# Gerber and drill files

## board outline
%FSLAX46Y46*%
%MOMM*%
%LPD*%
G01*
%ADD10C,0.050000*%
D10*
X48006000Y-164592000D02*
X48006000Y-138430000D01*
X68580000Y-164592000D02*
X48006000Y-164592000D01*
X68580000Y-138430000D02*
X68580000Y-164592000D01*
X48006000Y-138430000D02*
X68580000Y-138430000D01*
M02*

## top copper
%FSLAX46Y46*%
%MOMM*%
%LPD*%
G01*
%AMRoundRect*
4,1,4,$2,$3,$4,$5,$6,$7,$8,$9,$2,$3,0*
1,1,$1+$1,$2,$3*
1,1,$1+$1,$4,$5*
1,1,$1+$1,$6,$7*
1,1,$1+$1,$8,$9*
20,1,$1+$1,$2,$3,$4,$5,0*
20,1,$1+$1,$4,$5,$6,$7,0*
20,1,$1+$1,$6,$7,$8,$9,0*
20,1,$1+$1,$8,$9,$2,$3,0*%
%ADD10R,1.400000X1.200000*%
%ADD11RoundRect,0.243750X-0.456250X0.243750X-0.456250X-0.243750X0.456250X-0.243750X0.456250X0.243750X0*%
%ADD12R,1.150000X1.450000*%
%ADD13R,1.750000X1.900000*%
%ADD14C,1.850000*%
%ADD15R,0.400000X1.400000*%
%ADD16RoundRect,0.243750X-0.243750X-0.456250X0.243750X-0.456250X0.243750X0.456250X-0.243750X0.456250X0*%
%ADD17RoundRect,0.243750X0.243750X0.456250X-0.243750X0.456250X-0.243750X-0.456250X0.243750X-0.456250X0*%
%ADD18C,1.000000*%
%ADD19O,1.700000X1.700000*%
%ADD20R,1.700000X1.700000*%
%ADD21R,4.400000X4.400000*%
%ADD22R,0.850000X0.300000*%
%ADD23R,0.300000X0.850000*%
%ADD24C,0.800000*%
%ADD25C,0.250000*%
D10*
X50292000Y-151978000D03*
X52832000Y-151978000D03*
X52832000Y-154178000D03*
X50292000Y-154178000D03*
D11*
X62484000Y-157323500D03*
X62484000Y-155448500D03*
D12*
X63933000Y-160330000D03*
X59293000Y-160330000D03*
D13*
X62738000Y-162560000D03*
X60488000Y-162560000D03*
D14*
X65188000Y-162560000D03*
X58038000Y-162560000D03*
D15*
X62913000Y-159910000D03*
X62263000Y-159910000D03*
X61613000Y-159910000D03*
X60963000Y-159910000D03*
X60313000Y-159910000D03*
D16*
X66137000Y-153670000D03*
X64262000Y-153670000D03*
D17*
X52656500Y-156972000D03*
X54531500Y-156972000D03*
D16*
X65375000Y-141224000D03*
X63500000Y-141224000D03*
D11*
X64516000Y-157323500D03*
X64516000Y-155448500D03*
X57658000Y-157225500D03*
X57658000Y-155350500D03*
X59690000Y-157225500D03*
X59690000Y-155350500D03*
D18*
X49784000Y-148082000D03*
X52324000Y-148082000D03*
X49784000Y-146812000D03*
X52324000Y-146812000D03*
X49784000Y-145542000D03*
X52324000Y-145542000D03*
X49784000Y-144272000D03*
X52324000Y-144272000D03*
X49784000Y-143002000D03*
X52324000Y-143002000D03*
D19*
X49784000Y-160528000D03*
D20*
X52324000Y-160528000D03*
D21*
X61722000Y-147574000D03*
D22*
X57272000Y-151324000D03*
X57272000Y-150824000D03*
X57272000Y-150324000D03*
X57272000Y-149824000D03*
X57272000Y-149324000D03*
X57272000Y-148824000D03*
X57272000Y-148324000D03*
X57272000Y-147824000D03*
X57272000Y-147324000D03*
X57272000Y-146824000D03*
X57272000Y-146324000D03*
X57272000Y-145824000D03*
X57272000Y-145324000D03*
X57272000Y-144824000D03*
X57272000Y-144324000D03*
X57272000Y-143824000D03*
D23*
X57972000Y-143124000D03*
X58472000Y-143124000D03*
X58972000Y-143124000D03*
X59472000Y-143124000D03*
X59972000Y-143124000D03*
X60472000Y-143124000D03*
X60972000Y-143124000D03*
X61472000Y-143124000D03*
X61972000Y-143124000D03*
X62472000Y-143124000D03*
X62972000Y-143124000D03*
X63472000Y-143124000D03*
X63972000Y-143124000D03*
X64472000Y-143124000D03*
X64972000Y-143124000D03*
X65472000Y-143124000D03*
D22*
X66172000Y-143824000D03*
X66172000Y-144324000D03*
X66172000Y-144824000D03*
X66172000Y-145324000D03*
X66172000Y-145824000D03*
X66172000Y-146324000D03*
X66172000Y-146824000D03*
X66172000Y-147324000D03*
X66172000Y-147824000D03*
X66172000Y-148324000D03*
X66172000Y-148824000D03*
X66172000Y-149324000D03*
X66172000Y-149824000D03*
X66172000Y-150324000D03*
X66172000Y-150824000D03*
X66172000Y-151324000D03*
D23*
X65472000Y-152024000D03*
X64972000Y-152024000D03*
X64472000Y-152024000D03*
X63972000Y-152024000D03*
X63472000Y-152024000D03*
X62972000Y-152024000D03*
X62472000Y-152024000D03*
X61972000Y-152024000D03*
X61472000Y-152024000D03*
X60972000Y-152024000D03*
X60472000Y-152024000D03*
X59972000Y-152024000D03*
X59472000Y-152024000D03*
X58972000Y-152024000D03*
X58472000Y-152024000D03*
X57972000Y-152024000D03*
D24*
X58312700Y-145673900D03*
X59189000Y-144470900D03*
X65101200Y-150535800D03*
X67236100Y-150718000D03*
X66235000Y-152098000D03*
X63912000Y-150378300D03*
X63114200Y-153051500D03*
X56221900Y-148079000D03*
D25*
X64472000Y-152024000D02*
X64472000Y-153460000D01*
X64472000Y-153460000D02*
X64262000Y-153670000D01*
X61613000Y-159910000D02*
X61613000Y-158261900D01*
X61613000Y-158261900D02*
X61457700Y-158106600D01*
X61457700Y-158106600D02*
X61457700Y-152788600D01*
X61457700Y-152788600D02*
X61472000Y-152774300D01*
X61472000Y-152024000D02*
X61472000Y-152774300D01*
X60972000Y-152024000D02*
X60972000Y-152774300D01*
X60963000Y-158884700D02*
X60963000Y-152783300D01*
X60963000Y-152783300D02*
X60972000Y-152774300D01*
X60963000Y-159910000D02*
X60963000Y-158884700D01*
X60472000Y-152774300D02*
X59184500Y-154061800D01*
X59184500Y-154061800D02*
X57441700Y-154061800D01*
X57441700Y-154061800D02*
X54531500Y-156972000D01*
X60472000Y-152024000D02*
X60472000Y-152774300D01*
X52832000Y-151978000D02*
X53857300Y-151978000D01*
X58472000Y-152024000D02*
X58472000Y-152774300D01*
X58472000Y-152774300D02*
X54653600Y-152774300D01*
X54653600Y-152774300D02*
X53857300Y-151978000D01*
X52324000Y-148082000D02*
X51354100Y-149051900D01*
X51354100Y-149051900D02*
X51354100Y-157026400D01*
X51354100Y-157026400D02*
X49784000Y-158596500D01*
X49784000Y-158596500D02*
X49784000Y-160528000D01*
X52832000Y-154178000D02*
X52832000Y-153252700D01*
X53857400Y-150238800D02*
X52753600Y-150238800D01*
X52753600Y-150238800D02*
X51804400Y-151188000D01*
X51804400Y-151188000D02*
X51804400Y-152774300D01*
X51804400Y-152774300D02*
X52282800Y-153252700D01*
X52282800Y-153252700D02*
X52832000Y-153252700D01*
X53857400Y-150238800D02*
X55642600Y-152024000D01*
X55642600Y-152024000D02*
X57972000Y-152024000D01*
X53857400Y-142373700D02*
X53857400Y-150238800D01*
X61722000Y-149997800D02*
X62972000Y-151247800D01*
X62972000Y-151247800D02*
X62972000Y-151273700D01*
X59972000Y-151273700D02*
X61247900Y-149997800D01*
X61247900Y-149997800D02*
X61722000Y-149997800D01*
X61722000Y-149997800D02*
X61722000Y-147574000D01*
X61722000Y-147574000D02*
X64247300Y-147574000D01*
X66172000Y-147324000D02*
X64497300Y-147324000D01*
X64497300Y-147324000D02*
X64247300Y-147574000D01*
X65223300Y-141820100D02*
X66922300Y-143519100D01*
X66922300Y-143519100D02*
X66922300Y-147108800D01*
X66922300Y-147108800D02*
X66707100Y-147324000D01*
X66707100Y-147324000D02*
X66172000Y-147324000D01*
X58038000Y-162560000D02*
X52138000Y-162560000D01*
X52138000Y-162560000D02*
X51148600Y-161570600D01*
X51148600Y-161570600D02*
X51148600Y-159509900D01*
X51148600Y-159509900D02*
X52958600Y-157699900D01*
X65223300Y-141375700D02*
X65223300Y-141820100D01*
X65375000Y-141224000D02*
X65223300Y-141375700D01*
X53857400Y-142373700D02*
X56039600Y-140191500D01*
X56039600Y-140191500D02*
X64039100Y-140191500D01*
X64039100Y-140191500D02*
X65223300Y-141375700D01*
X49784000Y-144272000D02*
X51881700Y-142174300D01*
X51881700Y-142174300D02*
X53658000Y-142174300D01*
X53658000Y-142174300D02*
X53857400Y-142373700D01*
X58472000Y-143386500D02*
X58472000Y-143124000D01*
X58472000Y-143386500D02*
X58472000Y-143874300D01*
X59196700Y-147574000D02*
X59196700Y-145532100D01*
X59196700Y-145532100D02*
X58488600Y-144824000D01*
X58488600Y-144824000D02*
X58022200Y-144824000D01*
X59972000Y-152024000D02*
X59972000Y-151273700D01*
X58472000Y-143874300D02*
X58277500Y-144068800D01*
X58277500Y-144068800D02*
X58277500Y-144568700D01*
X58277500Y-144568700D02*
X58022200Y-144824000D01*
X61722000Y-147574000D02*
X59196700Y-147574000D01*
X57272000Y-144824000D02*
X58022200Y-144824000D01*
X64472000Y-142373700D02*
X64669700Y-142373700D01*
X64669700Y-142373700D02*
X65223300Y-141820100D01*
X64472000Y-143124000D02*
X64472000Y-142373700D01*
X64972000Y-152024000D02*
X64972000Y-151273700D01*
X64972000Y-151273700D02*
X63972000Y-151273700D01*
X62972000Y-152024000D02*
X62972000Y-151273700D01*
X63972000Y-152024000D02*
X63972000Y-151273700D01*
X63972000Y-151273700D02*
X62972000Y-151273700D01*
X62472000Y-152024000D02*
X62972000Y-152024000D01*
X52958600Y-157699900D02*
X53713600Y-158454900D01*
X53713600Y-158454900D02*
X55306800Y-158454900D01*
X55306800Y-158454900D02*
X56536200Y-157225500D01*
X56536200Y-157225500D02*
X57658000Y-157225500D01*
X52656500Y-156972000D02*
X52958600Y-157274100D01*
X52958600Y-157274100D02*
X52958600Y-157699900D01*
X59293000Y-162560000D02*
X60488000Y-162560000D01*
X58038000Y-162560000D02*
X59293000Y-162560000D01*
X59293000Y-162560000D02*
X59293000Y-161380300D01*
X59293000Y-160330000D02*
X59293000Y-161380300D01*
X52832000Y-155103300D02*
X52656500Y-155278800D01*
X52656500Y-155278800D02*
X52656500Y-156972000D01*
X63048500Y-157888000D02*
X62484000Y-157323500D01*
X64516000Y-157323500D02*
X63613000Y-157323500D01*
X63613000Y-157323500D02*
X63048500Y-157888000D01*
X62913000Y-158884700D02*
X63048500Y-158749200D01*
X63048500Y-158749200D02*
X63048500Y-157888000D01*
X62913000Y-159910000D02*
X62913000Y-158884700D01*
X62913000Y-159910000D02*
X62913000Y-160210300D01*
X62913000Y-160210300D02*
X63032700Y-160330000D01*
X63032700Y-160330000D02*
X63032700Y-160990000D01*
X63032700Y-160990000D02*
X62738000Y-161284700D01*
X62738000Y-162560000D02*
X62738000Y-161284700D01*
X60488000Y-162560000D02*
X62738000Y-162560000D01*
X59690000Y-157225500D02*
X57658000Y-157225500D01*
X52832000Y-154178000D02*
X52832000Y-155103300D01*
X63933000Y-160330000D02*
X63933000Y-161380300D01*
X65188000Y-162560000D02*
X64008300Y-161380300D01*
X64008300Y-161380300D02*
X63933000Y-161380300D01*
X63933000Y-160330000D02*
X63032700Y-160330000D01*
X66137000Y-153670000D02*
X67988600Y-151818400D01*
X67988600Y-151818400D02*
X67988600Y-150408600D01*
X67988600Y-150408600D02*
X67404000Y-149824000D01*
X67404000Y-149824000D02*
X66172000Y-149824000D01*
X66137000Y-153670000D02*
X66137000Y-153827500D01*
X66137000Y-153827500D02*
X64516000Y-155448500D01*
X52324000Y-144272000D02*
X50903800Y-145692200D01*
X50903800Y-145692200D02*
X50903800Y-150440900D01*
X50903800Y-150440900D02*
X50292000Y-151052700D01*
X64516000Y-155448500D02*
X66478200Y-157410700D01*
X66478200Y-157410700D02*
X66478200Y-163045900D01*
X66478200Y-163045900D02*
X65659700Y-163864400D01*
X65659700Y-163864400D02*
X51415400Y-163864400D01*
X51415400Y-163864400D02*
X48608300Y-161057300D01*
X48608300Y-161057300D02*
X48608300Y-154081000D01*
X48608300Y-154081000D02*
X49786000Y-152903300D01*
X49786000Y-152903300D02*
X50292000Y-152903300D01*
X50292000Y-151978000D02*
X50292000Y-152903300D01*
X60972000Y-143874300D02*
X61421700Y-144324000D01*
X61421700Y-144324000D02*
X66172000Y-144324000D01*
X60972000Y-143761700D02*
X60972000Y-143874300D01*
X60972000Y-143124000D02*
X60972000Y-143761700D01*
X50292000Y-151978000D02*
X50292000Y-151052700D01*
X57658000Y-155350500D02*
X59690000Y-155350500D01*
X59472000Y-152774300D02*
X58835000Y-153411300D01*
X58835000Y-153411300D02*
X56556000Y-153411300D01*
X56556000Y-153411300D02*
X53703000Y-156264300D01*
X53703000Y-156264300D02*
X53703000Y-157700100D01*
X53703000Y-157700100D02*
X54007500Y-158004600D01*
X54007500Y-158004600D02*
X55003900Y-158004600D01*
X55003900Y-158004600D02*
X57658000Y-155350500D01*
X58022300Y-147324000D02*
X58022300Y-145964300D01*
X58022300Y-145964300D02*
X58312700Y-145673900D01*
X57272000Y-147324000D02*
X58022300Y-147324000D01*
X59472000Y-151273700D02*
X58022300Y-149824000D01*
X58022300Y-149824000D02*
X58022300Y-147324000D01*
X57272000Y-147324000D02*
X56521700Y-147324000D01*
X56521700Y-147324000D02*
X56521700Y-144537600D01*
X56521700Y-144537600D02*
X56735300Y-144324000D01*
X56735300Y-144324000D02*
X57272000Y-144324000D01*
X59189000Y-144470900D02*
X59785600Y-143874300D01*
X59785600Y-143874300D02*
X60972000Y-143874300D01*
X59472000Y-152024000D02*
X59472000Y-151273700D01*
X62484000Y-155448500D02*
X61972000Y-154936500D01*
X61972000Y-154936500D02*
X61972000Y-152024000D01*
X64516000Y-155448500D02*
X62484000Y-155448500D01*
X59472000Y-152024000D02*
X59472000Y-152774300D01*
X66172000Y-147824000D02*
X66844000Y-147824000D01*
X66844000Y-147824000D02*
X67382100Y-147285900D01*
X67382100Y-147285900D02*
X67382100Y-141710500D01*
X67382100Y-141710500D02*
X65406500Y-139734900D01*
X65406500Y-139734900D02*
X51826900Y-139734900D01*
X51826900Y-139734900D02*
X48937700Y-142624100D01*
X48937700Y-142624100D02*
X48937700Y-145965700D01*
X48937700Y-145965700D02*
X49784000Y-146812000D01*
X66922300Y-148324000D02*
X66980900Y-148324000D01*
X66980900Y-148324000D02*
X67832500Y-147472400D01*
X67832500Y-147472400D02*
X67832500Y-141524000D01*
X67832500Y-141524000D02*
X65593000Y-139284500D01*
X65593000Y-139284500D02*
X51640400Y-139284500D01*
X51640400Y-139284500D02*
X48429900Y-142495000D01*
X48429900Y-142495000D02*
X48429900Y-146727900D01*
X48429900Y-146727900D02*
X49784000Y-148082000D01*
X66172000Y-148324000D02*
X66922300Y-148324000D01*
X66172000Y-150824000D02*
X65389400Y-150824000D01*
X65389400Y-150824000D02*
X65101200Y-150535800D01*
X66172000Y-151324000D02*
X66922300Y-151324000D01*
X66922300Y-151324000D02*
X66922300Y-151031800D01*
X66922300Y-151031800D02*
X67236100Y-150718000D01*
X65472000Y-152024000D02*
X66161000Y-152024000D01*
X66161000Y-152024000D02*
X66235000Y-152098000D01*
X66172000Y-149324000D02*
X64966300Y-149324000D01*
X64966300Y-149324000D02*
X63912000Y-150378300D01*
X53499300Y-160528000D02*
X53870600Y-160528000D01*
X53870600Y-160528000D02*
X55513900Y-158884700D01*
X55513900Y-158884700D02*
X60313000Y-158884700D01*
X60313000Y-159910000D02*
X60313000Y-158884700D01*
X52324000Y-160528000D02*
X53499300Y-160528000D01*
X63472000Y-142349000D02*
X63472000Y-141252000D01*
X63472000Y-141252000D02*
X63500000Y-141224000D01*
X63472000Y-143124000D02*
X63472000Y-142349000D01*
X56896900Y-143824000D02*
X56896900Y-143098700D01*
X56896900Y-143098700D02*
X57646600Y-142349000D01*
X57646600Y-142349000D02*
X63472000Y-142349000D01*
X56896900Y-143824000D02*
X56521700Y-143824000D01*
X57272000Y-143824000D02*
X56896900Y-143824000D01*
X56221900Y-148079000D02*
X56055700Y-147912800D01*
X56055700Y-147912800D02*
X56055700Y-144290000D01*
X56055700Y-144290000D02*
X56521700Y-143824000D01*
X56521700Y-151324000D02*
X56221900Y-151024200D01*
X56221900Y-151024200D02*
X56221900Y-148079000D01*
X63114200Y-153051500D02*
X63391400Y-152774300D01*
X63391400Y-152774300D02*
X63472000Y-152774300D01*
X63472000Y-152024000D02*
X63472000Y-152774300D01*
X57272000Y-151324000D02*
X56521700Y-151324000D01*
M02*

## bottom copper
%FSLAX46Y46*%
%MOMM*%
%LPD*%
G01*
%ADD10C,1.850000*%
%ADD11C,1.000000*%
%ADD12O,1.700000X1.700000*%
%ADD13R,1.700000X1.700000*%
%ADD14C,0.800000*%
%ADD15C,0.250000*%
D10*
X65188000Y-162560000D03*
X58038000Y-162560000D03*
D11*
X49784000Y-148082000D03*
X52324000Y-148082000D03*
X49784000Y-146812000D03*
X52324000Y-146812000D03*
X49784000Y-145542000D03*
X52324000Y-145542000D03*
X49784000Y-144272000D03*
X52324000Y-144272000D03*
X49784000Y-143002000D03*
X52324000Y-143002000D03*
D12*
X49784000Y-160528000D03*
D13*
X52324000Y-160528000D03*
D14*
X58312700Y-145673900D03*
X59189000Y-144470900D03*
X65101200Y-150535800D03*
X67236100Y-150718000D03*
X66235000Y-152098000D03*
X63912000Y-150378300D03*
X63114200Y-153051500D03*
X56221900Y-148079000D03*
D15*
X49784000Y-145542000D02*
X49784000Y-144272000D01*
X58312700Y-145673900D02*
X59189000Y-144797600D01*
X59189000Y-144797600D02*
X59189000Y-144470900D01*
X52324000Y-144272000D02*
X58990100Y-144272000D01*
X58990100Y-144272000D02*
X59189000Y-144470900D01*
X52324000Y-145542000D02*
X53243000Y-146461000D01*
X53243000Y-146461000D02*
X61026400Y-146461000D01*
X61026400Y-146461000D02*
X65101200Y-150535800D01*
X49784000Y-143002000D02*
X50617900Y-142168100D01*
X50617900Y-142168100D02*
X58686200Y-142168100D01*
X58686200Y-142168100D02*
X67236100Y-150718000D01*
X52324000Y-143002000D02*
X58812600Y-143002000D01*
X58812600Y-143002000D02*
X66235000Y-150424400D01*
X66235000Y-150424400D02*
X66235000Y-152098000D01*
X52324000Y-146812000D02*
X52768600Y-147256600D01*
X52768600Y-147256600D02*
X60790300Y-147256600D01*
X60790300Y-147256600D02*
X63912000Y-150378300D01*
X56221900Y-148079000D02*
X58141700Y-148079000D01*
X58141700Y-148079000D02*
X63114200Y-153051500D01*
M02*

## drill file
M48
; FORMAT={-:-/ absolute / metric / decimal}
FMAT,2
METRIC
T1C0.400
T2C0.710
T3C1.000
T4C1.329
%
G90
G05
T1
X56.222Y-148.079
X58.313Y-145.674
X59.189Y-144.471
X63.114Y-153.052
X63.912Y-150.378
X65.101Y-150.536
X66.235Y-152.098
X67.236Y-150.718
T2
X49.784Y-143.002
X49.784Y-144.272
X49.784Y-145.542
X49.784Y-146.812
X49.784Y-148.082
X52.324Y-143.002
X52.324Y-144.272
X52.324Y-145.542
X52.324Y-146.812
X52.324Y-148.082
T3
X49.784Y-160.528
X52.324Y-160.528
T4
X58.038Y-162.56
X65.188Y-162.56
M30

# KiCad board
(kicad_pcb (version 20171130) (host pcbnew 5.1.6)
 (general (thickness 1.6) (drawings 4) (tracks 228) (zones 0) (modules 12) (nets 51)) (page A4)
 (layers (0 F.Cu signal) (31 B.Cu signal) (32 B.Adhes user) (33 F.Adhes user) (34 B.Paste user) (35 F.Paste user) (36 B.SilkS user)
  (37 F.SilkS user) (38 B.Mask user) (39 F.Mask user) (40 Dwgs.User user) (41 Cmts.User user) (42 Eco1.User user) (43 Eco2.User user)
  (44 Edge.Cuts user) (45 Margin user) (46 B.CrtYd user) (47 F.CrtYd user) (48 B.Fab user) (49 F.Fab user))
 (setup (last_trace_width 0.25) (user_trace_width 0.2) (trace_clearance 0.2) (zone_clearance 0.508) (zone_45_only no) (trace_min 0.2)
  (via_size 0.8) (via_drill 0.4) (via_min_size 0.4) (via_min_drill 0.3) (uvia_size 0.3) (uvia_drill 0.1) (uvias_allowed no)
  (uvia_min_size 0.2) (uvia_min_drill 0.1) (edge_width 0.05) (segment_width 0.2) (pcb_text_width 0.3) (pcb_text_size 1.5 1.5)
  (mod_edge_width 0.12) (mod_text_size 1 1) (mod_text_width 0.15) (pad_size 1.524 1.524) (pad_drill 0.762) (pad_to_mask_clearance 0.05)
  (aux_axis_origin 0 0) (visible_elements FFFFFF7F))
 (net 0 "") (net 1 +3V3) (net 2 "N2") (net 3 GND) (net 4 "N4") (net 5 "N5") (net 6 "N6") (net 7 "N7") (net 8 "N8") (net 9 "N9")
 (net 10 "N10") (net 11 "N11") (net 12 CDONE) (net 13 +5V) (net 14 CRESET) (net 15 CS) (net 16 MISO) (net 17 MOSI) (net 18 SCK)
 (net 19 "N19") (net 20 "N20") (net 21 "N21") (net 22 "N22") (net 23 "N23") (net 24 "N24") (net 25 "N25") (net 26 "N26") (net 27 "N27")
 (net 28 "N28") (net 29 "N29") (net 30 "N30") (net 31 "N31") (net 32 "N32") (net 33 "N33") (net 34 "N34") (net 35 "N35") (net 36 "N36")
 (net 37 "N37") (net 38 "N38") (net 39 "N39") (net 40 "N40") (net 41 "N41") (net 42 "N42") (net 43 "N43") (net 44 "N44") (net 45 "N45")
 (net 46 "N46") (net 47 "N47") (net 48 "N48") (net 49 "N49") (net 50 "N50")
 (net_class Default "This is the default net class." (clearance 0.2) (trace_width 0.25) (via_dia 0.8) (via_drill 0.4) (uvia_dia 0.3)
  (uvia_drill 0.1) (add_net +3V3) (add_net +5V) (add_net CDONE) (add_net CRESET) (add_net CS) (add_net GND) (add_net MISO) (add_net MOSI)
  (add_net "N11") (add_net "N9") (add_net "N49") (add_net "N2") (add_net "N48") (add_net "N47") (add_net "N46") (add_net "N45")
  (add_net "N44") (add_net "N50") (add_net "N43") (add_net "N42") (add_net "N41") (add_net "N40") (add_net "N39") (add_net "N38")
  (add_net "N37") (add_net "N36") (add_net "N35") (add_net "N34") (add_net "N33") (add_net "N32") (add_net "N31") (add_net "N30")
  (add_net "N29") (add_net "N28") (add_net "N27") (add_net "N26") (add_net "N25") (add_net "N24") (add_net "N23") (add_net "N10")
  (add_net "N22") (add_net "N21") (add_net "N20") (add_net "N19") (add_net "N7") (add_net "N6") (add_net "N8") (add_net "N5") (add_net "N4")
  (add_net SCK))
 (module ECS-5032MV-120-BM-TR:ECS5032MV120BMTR (layer F.Cu) (at 51.562 153.078)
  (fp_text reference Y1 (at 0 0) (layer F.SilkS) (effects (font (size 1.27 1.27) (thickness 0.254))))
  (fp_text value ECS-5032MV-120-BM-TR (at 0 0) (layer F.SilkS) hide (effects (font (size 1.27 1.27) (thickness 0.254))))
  (pad 4 smd rect (at -1.27 -1.1 90) (size 1.2 1.4) (layers F.Cu F.Paste F.Mask) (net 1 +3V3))
  (pad 3 smd rect (at 1.27 -1.1 90) (size 1.2 1.4) (layers F.Cu F.Paste F.Mask) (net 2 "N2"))
  (pad 2 smd rect (at 1.27 1.1 90) (size 1.2 1.4) (layers F.Cu F.Paste F.Mask) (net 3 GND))
  (pad 1 smd rect (at -1.27 1.1 90) (size 1.2 1.4) (layers F.Cu F.Paste F.Mask) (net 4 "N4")))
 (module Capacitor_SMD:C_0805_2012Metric (layer F.Cu) (at 62.484 156.386 270)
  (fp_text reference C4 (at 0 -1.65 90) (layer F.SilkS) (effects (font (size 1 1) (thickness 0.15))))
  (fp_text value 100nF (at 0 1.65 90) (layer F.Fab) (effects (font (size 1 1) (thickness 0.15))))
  (pad 2 smd roundrect (at 0.9375 0 270) (size 0.975 1.4) (layers F.Cu F.Paste F.Mask) (roundrect_rratio 0.25) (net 3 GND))
  (pad 1 smd roundrect (at -0.9375 0 270) (size 0.975 1.4) (layers F.Cu F.Paste F.Mask) (roundrect_rratio 0.25) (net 1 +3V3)))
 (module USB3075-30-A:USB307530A (layer F.Cu) (at 61.613 162.56)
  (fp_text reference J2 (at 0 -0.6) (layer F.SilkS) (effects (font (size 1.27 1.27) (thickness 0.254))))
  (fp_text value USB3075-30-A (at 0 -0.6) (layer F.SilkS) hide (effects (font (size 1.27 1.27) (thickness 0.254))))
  (pad MP4 smd rect (at 2.32 -2.23) (size 1.15 1.45) (layers F.Cu F.Paste F.Mask) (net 3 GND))
  (pad MP3 smd rect (at -2.32 -2.23) (size 1.15 1.45) (layers F.Cu F.Paste F.Mask) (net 3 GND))
  (pad MP2 smd rect (at 1.125 0) (size 1.75 1.9) (layers F.Cu F.Paste F.Mask) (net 3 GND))
  (pad MP1 smd rect (at -1.125 0) (size 1.75 1.9) (layers F.Cu F.Paste F.Mask) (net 3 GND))
  (pad MH2 thru_hole circle (at 3.575 0) (size 1.85 1.85) (drill 1.3285) (layers *.Cu *.Mask) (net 3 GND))
  (pad MH1 thru_hole circle (at -3.575 0) (size 1.85 1.85) (drill 1.3285) (layers *.Cu *.Mask) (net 3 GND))
  (pad 5 smd rect (at 1.3 -2.65) (size 0.4 1.4) (layers F.Cu F.Paste F.Mask) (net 3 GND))
  (pad 4 smd rect (at 0.65 -2.65) (size 0.4 1.4) (layers F.Cu F.Paste F.Mask) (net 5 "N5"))
  (pad 3 smd rect (at 0 -2.65) (size 0.4 1.4) (layers F.Cu F.Paste F.Mask) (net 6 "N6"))
  (pad 2 smd rect (at -0.65 -2.65) (size 0.4 1.4) (layers F.Cu F.Paste F.Mask) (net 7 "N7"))
  (pad 1 smd rect (at -1.3 -2.65) (size 0.4 1.4) (layers F.Cu F.Paste F.Mask) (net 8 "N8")))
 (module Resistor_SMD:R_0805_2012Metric (layer F.Cu) (at 65.1995 153.67)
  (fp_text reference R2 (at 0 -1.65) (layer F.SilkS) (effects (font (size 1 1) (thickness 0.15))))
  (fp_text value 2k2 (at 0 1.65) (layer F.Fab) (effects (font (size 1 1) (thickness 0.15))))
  (pad 2 smd roundrect (at 0.9375 0) (size 0.975 1.4) (layers F.Cu F.Paste F.Mask) (roundrect_rratio 0.25) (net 1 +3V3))
  (pad 1 smd roundrect (at -0.9375 0) (size 0.975 1.4) (layers F.Cu F.Paste F.Mask) (roundrect_rratio 0.25) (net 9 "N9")))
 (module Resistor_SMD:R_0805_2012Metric (layer F.Cu) (at 53.594 156.972 180)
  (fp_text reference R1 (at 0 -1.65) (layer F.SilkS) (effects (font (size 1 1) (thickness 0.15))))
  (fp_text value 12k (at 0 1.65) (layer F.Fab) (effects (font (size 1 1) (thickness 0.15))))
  (pad 2 smd roundrect (at 0.9375 0 180) (size 0.975 1.4) (layers F.Cu F.Paste F.Mask) (roundrect_rratio 0.25) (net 3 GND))
  (pad 1 smd roundrect (at -0.9375 0 180) (size 0.975 1.4) (layers F.Cu F.Paste F.Mask) (roundrect_rratio 0.25) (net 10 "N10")))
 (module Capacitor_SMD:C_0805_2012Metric (layer F.Cu) (at 64.4375 141.224)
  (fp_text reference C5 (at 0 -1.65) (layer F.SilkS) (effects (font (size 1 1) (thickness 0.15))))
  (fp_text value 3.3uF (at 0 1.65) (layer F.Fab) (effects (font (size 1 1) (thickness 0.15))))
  (pad 2 smd roundrect (at 0.9375 0) (size 0.975 1.4) (layers F.Cu F.Paste F.Mask) (roundrect_rratio 0.25) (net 3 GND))
  (pad 1 smd roundrect (at -0.9375 0) (size 0.975 1.4) (layers F.Cu F.Paste F.Mask) (roundrect_rratio 0.25) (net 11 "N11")))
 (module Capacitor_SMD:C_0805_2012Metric (layer F.Cu) (at 64.516 156.386 270)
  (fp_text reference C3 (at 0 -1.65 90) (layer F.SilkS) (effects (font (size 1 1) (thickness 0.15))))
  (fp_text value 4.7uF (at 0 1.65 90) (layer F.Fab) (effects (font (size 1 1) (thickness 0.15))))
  (pad 2 smd roundrect (at 0.9375 0 270) (size 0.975 1.4) (layers F.Cu F.Paste F.Mask) (roundrect_rratio 0.25) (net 3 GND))
  (pad 1 smd roundrect (at -0.9375 0 270) (size 0.975 1.4) (layers F.Cu F.Paste F.Mask) (roundrect_rratio 0.25) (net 1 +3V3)))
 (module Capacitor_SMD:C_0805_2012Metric (layer F.Cu) (at 57.658 156.288 270)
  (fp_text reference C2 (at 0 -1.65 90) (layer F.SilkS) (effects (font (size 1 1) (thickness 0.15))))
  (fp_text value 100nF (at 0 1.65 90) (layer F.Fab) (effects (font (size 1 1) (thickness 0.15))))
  (pad 2 smd roundrect (at 0.9375 0 270) (size 0.975 1.4) (layers F.Cu F.Paste F.Mask) (roundrect_rratio 0.25) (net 3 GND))
  (pad 1 smd roundrect (at -0.9375 0 270) (size 0.975 1.4) (layers F.Cu F.Paste F.Mask) (roundrect_rratio 0.25) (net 1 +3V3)))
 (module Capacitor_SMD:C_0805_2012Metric (layer F.Cu) (at 59.69 156.288 270)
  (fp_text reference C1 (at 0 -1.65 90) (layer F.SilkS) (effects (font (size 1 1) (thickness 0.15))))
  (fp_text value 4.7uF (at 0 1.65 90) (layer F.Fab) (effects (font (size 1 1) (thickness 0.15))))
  (pad 2 smd roundrect (at 0.9375 0 270) (size 0.975 1.4) (layers F.Cu F.Paste F.Mask) (roundrect_rratio 0.25) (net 3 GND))
  (pad 1 smd roundrect (at -0.9375 0 270) (size 0.975 1.4) (layers F.Cu F.Paste F.Mask) (roundrect_rratio 0.25) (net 1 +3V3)))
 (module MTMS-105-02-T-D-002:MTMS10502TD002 (layer B.Cu) (at 52.324 143.002 270)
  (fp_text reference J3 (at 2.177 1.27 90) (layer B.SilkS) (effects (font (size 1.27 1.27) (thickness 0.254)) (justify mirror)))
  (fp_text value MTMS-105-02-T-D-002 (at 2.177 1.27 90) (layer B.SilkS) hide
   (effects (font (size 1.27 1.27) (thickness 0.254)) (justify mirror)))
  (pad 10 thru_hole circle (at 5.08 2.54 270) (size 1 1) (drill 0.71) (layers *.Cu *.Mask) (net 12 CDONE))
  (pad 9 thru_hole circle (at 5.08 0 270) (size 1 1) (drill 0.71) (layers *.Cu *.Mask) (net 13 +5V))
  (pad 8 thru_hole circle (at 3.81 2.54 270) (size 1 1) (drill 0.71) (layers *.Cu *.Mask) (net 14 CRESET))
  (pad 7 thru_hole circle (at 3.81 0 270) (size 1 1) (drill 0.71) (layers *.Cu *.Mask) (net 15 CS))
  (pad 6 thru_hole circle (at 2.54 2.54 270) (size 1 1) (drill 0.71) (layers *.Cu *.Mask) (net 3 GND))
  (pad 5 thru_hole circle (at 2.54 0 270) (size 1 1) (drill 0.71) (layers *.Cu *.Mask) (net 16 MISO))
  (pad 4 thru_hole circle (at 1.27 2.54 270) (size 1 1) (drill 0.71) (layers *.Cu *.Mask) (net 3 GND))
  (pad 3 thru_hole circle (at 1.27 0 270) (size 1 1) (drill 0.71) (layers *.Cu *.Mask) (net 1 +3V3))
  (pad 2 thru_hole circle (at 0 2.54 270) (size 1 1) (drill 0.71) (layers *.Cu *.Mask) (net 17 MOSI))
  (pad 1 thru_hole circle (at 0 0 270) (size 1 1) (drill 0.71) (layers *.Cu *.Mask) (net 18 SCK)))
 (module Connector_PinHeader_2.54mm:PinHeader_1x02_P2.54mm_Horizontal (layer F.Cu) (at 52.324 160.528 270)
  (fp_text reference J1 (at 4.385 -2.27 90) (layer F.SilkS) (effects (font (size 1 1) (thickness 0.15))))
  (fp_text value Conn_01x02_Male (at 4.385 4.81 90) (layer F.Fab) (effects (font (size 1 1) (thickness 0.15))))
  (pad 2 thru_hole oval (at 0 2.54 270) (size 1.7 1.7) (drill 1) (layers *.Cu *.Mask) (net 13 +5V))
  (pad 1 thru_hole rect (at 0 0 270) (size 1.7 1.7) (drill 1) (layers *.Cu *.Mask) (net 8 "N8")))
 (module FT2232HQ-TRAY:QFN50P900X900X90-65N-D (layer F.Cu) (at 61.722 147.574 90)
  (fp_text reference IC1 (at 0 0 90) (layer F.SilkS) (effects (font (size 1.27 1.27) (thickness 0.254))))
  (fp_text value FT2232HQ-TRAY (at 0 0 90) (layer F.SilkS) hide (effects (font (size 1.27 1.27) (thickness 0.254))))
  (pad 65 smd rect (at 0 0 90) (size 4.4 4.4) (layers F.Cu F.Paste F.Mask) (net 3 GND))
  (pad 64 smd rect (at -3.75 -4.45 90) (size 0.3 0.85) (layers F.Cu F.Paste F.Mask) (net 11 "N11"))
  (pad 63 smd rect (at -3.25 -4.45 90) (size 0.3 0.85) (layers F.Cu F.Paste F.Mask) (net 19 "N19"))
  (pad 62 smd rect (at -2.75 -4.45 90) (size 0.3 0.85) (layers F.Cu F.Paste F.Mask) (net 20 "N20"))
  (pad 61 smd rect (at -2.25 -4.45 90) (size 0.3 0.85) (layers F.Cu F.Paste F.Mask) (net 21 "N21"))
  (pad 60 smd rect (at -1.75 -4.45 90) (size 0.3 0.85) (layers F.Cu F.Paste F.Mask) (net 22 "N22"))
  (pad 59 smd rect (at -1.25 -4.45 90) (size 0.3 0.85) (layers F.Cu F.Paste F.Mask) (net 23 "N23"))
  (pad 58 smd rect (at -0.75 -4.45 90) (size 0.3 0.85) (layers F.Cu F.Paste F.Mask) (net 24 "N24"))
  (pad 57 smd rect (at -0.25 -4.45 90) (size 0.3 0.85) (layers F.Cu F.Paste F.Mask) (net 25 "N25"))
  (pad 56 smd rect (at 0.25 -4.45 90) (size 0.3 0.85) (layers F.Cu F.Paste F.Mask) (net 1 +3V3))
  (pad 55 smd rect (at 0.75 -4.45 90) (size 0.3 0.85) (layers F.Cu F.Paste F.Mask) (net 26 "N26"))
  (pad 54 smd rect (at 1.25 -4.45 90) (size 0.3 0.85) (layers F.Cu F.Paste F.Mask) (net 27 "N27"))
  (pad 53 smd rect (at 1.75 -4.45 90) (size 0.3 0.85) (layers F.Cu F.Paste F.Mask) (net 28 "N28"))
  (pad 52 smd rect (at 2.25 -4.45 90) (size 0.3 0.85) (layers F.Cu F.Paste F.Mask) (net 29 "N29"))
  (pad 51 smd rect (at 2.75 -4.45 90) (size 0.3 0.85) (layers F.Cu F.Paste F.Mask) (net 3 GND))
  (pad 50 smd rect (at 3.25 -4.45 90) (size 0.3 0.85) (layers F.Cu F.Paste F.Mask) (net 1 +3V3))
  (pad 49 smd rect (at 3.75 -4.45 90) (size 0.3 0.85) (layers F.Cu F.Paste F.Mask) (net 11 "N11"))
  (pad 48 smd rect (at 4.45 -3.75 180) (size 0.3 0.85) (layers F.Cu F.Paste F.Mask) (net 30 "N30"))
  (pad 47 smd rect (at 4.45 -3.25 180) (size 0.3 0.85) (layers F.Cu F.Paste F.Mask) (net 3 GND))
  (pad 46 smd rect (at 4.45 -2.75 180) (size 0.3 0.85) (layers F.Cu F.Paste F.Mask) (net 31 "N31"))
  (pad 45 smd rect (at 4.45 -2.25 180) (size 0.3 0.85) (layers F.Cu F.Paste F.Mask) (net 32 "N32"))
  (pad 44 smd rect (at 4.45 -1.75 180) (size 0.3 0.85) (layers F.Cu F.Paste F.Mask) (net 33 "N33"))
  (pad 43 smd rect (at 4.45 -1.25 180) (size 0.3 0.85) (layers F.Cu F.Paste F.Mask) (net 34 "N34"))
  (pad 42 smd rect (at 4.45 -0.75 180) (size 0.3 0.85) (layers F.Cu F.Paste F.Mask) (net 1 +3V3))
  (pad 41 smd rect (at 4.45 -0.25 180) (size 0.3 0.85) (layers F.Cu F.Paste F.Mask) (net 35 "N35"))
  (pad 40 smd rect (at 4.45 0.25 180) (size 0.3 0.85) (layers F.Cu F.Paste F.Mask) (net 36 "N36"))
  (pad 39 smd rect (at 4.45 0.75 180) (size 0.3 0.85) (layers F.Cu F.Paste F.Mask) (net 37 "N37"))
  (pad 38 smd rect (at 4.45 1.25 180) (size 0.3 0.85) (layers F.Cu F.Paste F.Mask) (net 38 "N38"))
  (pad 37 smd rect (at 4.45 1.75 180) (size 0.3 0.85) (layers F.Cu F.Paste F.Mask) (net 11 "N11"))
  (pad 36 smd rect (at 4.45 2.25 180) (size 0.3 0.85) (layers F.Cu F.Paste F.Mask) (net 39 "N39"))
  (pad 35 smd rect (at 4.45 2.75 180) (size 0.3 0.85) (layers F.Cu F.Paste F.Mask) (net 3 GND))
  (pad 34 smd rect (at 4.45 3.25 180) (size 0.3 0.85) (layers F.Cu F.Paste F.Mask) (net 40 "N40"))
  (pad 33 smd rect (at 4.45 3.75 180) (size 0.3 0.85) (layers F.Cu F.Paste F.Mask) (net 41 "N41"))
  (pad 32 smd rect (at 3.75 4.45 90) (size 0.3 0.85) (layers F.Cu F.Paste F.Mask) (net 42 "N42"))
  (pad 31 smd rect (at 3.25 4.45 90) (size 0.3 0.85) (layers F.Cu F.Paste F.Mask) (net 1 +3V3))
  (pad 30 smd rect (at 2.75 4.45 90) (size 0.3 0.85) (layers F.Cu F.Paste F.Mask) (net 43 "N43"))
  (pad 29 smd rect (at 2.25 4.45 90) (size 0.3 0.85) (layers F.Cu F.Paste F.Mask) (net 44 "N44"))
  (pad 28 smd rect (at 1.75 4.45 90) (size 0.3 0.85) (layers F.Cu F.Paste F.Mask) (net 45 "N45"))
  (pad 27 smd rect (at 1.25 4.45 90) (size 0.3 0.85) (layers F.Cu F.Paste F.Mask) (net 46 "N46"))
  (pad 26 smd rect (at 0.75 4.45 90) (size 0.3 0.85) (layers F.Cu F.Paste F.Mask) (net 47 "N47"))
  (pad 25 smd rect (at 0.25 4.45 90) (size 0.3 0.85) (layers F.Cu F.Paste F.Mask) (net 3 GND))
  (pad 24 smd rect (at -0.25 4.45 90) (size 0.3 0.85) (layers F.Cu F.Paste F.Mask) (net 14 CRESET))
  (pad 23 smd rect (at -0.75 4.45 90) (size 0.3 0.85) (layers F.Cu F.Paste F.Mask) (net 12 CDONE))
  (pad 22 smd rect (at -1.25 4.45 90) (size 0.3 0.85) (layers F.Cu F.Paste F.Mask) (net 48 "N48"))
  (pad 21 smd rect (at -1.75 4.45 90) (size 0.3 0.85) (layers F.Cu F.Paste F.Mask) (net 15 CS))
  (pad 20 smd rect (at -2.25 4.45 90) (size 0.3 0.85) (layers F.Cu F.Paste F.Mask) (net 1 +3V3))
  (pad 19 smd rect (at -2.75 4.45 90) (size 0.3 0.85) (layers F.Cu F.Paste F.Mask) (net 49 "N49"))
  (pad 18 smd rect (at -3.25 4.45 90) (size 0.3 0.85) (layers F.Cu F.Paste F.Mask) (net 16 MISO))
  (pad 17 smd rect (at -3.75 4.45 90) (size 0.3 0.85) (layers F.Cu F.Paste F.Mask) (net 17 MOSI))
  (pad 16 smd rect (at -4.45 3.75 180) (size 0.3 0.85) (layers F.Cu F.Paste F.Mask) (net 18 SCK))
  (pad 15 smd rect (at -4.45 3.25 180) (size 0.3 0.85) (layers F.Cu F.Paste F.Mask) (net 3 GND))
  (pad 14 smd rect (at -4.45 2.75 180) (size 0.3 0.85) (layers F.Cu F.Paste F.Mask) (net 9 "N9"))
  (pad 13 smd rect (at -4.45 2.25 180) (size 0.3 0.85) (layers F.Cu F.Paste F.Mask) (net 3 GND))
  (pad 12 smd rect (at -4.45 1.75 180) (size 0.3 0.85) (layers F.Cu F.Paste F.Mask) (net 11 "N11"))
  (pad 11 smd rect (at -4.45 1.25 180) (size 0.3 0.85) (layers F.Cu F.Paste F.Mask) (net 3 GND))
  (pad 10 smd rect (at -4.45 0.75 180) (size 0.3 0.85) (layers F.Cu F.Paste F.Mask) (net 3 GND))
  (pad 9 smd rect (at -4.45 0.25 180) (size 0.3 0.85) (layers F.Cu F.Paste F.Mask) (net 1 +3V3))
  (pad 8 smd rect (at -4.45 -0.25 180) (size 0.3 0.85) (layers F.Cu F.Paste F.Mask) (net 6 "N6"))
  (pad 7 smd rect (at -4.45 -0.75 180) (size 0.3 0.85) (layers F.Cu F.Paste F.Mask) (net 7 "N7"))
  (pad 6 smd rect (at -4.45 -1.25 180) (size 0.3 0.85) (layers F.Cu F.Paste F.Mask) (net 10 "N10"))
  (pad 5 smd rect (at -4.45 -1.75 180) (size 0.3 0.85) (layers F.Cu F.Paste F.Mask) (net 3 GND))
  (pad 4 smd rect (at -4.45 -2.25 180) (size 0.3 0.85) (layers F.Cu F.Paste F.Mask) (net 1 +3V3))
  (pad 3 smd rect (at -4.45 -2.75 180) (size 0.3 0.85) (layers F.Cu F.Paste F.Mask) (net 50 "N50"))
  (pad 2 smd rect (at -4.45 -3.25 180) (size 0.3 0.85) (layers F.Cu F.Paste F.Mask) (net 2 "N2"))
  (pad 1 smd rect (at -4.45 -3.75 180) (size 0.3 0.85) (layers F.Cu F.Paste F.Mask) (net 3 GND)))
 (gr_line (start 48.006 164.592) (end 48.006 138.43) (layer Edge.Cuts) (width 0.05))
 (gr_line (start 68.58 164.592) (end 48.006 164.592) (layer Edge.Cuts) (width 0.05))
 (gr_line (start 68.58 138.43) (end 68.58 164.592) (layer Edge.Cuts) (width 0.05))
 (gr_line (start 48.006 138.43) (end 68.58 138.43) (layer Edge.Cuts) (width 0.05))
 (segment (start 64.472 152.024) (end 64.472 153.46) (width 0.25) (layer F.Cu) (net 9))
 (segment (start 64.472 153.46) (end 64.262 153.67) (width 0.25) (layer F.Cu) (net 9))
 (segment (start 61.613 159.91) (end 61.613 158.2619) (width 0.25) (layer F.Cu) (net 6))
 (segment (start 61.613 158.2619) (end 61.4577 158.1066) (width 0.25) (layer F.Cu) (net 6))
 (segment (start 61.4577 158.1066) (end 61.4577 152.7886) (width 0.25) (layer F.Cu) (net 6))
 (segment (start 61.4577 152.7886) (end 61.472 152.7743) (width 0.25) (layer F.Cu) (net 6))
 (segment (start 61.472 152.024) (end 61.472 152.7743) (width 0.25) (layer F.Cu) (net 6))
 (segment (start 60.972 152.024) (end 60.972 152.7743) (width 0.25) (layer F.Cu) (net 7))
 (segment (start 60.963 158.8847) (end 60.963 152.7833) (width 0.25) (layer F.Cu) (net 7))
 (segment (start 60.963 152.7833) (end 60.972 152.7743) (width 0.25) (layer F.Cu) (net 7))
 (segment (start 60.963 159.91) (end 60.963 158.8847) (width 0.25) (layer F.Cu) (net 7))
 (segment (start 60.472 152.7743) (end 59.1845 154.0618) (width 0.25) (layer F.Cu) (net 10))
 (segment (start 59.1845 154.0618) (end 57.4417 154.0618) (width 0.25) (layer F.Cu) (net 10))
 (segment (start 57.4417 154.0618) (end 54.5315 156.972) (width 0.25) (layer F.Cu) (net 10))
 (segment (start 60.472 152.024) (end 60.472 152.7743) (width 0.25) (layer F.Cu) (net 10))
 (segment (start 52.832 151.978) (end 53.8573 151.978) (width 0.25) (layer F.Cu) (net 2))
 (segment (start 58.472 152.024) (end 58.472 152.7743) (width 0.25) (layer F.Cu) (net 2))
 (segment (start 58.472 152.7743) (end 54.6536 152.7743) (width 0.25) (layer F.Cu) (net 2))
 (segment (start 54.6536 152.7743) (end 53.8573 151.978) (width 0.25) (layer F.Cu) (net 2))
 (segment (start 52.324 148.082) (end 51.3541 149.0519) (width 0.25) (layer F.Cu) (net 13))
 (segment (start 51.3541 149.0519) (end 51.3541 157.0264) (width 0.25) (layer F.Cu) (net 13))
 (segment (start 51.3541 157.0264) (end 49.784 158.5965) (width 0.25) (layer F.Cu) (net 13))
 (segment (start 49.784 158.5965) (end 49.784 160.528) (width 0.25) (layer F.Cu) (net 13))
 (segment (start 52.832 154.178) (end 52.832 153.2527) (width 0.25) (layer F.Cu) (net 3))
 (segment (start 53.8574 150.2388) (end 52.7536 150.2388) (width 0.25) (layer F.Cu) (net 3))
 (segment (start 52.7536 150.2388) (end 51.8044 151.188) (width 0.25) (layer F.Cu) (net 3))
 (segment (start 51.8044 151.188) (end 51.8044 152.7743) (width 0.25) (layer F.Cu) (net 3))
 (segment (start 51.8044 152.7743) (end 52.2828 153.2527) (width 0.25) (layer F.Cu) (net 3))
 (segment (start 52.2828 153.2527) (end 52.832 153.2527) (width 0.25) (layer F.Cu) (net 3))
 (segment (start 53.8574 150.2388) (end 55.6426 152.024) (width 0.25) (layer F.Cu) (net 3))
 (segment (start 55.6426 152.024) (end 57.972 152.024) (width 0.25) (layer F.Cu) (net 3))
 (segment (start 53.8574 142.3737) (end 53.8574 150.2388) (width 0.25) (layer F.Cu) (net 3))
 (segment (start 61.722 149.9978) (end 62.972 151.2478) (width 0.25) (layer F.Cu) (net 3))
 (segment (start 62.972 151.2478) (end 62.972 151.2737) (width 0.25) (layer F.Cu) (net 3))
 (segment (start 59.972 151.2737) (end 61.2479 149.9978) (width 0.25) (layer F.Cu) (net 3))
 (segment (start 61.2479 149.9978) (end 61.722 149.9978) (width 0.25) (layer F.Cu) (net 3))
 (segment (start 61.722 149.9978) (end 61.722 147.574) (width 0.25) (layer F.Cu) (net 3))
 (segment (start 61.722 147.574) (end 64.2473 147.574) (width 0.25) (layer F.Cu) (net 3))
 (segment (start 66.172 147.324) (end 64.4973 147.324) (width 0.25) (layer F.Cu) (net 3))
 (segment (start 64.4973 147.324) (end 64.2473 147.574) (width 0.25) (layer F.Cu) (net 3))
 (segment (start 65.2233 141.8201) (end 66.9223 143.5191) (width 0.25) (layer F.Cu) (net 3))
 (segment (start 66.9223 143.5191) (end 66.9223 147.1088) (width 0.25) (layer F.Cu) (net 3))
 (segment (start 66.9223 147.1088) (end 66.7071 147.324) (width 0.25) (layer F.Cu) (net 3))
 (segment (start 66.7071 147.324) (end 66.172 147.324) (width 0.25) (layer F.Cu) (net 3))
 (segment (start 58.038 162.56) (end 52.138 162.56) (width 0.25) (layer F.Cu) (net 3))
 (segment (start 52.138 162.56) (end 51.1486 161.5706) (width 0.25) (layer F.Cu) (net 3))
 (segment (start 51.1486 161.5706) (end 51.1486 159.5099) (width 0.25) (layer F.Cu) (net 3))
 (segment (start 51.1486 159.5099) (end 52.9586 157.6999) (width 0.25) (layer F.Cu) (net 3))
 (segment (start 65.2233 141.3757) (end 65.2233 141.8201) (width 0.25) (layer F.Cu) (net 3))
 (segment (start 65.375 141.224) (end 65.2233 141.3757) (width 0.25) (layer F.Cu) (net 3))
 (segment (start 53.8574 142.3737) (end 56.0396 140.1915) (width 0.25) (layer F.Cu) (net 3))
 (segment (start 56.0396 140.1915) (end 64.0391 140.1915) (width 0.25) (layer F.Cu) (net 3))
 (segment (start 64.0391 140.1915) (end 65.2233 141.3757) (width 0.25) (layer F.Cu) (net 3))
 (segment (start 49.784 144.272) (end 51.8817 142.1743) (width 0.25) (layer F.Cu) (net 3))
 (segment (start 51.8817 142.1743) (end 53.658 142.1743) (width 0.25) (layer F.Cu) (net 3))
 (segment (start 53.658 142.1743) (end 53.8574 142.3737) (width 0.25) (layer F.Cu) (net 3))
 (segment (start 58.472 143.3865) (end 58.472 143.124) (width 0.25) (layer F.Cu) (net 3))
 (segment (start 58.472 143.3865) (end 58.472 143.8743) (width 0.25) (layer F.Cu) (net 3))
 (segment (start 49.784 145.542) (end 49.784 144.272) (width 0.25) (layer B.Cu) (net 3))
 (segment (start 59.1967 147.574) (end 59.1967 145.5321) (width 0.25) (layer F.Cu) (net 3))
 (segment (start 59.1967 145.5321) (end 58.4886 144.824) (width 0.25) (layer F.Cu) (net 3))
 (segment (start 58.4886 144.824) (end 58.0222 144.824) (width 0.25) (layer F.Cu) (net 3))
 (segment (start 59.972 152.024) (end 59.972 151.2737) (width 0.25) (layer F.Cu) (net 3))
 (segment (start 58.472 143.8743) (end 58.2775 144.0688) (width 0.25) (layer F.Cu) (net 3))
 (segment (start 58.2775 144.0688) (end 58.2775 144.5687) (width 0.25) (layer F.Cu) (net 3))
 (segment (start 58.2775 144.5687) (end 58.0222 144.824) (width 0.25) (layer F.Cu) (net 3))
 (segment (start 61.722 147.574) (end 59.1967 147.574) (width 0.25) (layer F.Cu) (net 3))
 (segment (start 57.272 144.824) (end 58.0222 144.824) (width 0.25) (layer F.Cu) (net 3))
 (segment (start 64.472 142.3737) (end 64.6697 142.3737) (width 0.25) (layer F.Cu) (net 3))
 (segment (start 64.6697 142.3737) (end 65.2233 141.8201) (width 0.25) (layer F.Cu) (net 3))
 (segment (start 64.472 143.124) (end 64.472 142.3737) (width 0.25) (layer F.Cu) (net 3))
 (segment (start 64.972 152.024) (end 64.972 151.2737) (width 0.25) (layer F.Cu) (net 3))
 (segment (start 64.972 151.2737) (end 63.972 151.2737) (width 0.25) (layer F.Cu) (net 3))
 (segment (start 62.972 152.024) (end 62.972 151.2737) (width 0.25) (layer F.Cu) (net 3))
 (segment (start 63.972 152.024) (end 63.972 151.2737) (width 0.25) (layer F.Cu) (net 3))
 (segment (start 63.972 151.2737) (end 62.972 151.2737) (width 0.25) (layer F.Cu) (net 3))
 (segment (start 62.472 152.024) (end 62.972 152.024) (width 0.25) (layer F.Cu) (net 3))
 (segment (start 52.9586 157.6999) (end 53.7136 158.4549) (width 0.25) (layer F.Cu) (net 3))
 (segment (start 53.7136 158.4549) (end 55.3068 158.4549) (width 0.25) (layer F.Cu) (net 3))
 (segment (start 55.3068 158.4549) (end 56.5362 157.2255) (width 0.25) (layer F.Cu) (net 3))
 (segment (start 56.5362 157.2255) (end 57.658 157.2255) (width 0.25) (layer F.Cu) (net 3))
 (segment (start 52.6565 156.972) (end 52.9586 157.2741) (width 0.25) (layer F.Cu) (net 3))
 (segment (start 52.9586 157.2741) (end 52.9586 157.6999) (width 0.25) (layer F.Cu) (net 3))
 (segment (start 59.293 162.56) (end 60.488 162.56) (width 0.25) (layer F.Cu) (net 3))
 (segment (start 58.038 162.56) (end 59.293 162.56) (width 0.25) (layer F.Cu) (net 3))
 (segment (start 59.293 162.56) (end 59.293 161.3803) (width 0.25) (layer F.Cu) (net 3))
 (segment (start 59.293 160.33) (end 59.293 161.3803) (width 0.25) (layer F.Cu) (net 3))
 (segment (start 52.832 155.1033) (end 52.6565 155.2788) (width 0.25) (layer F.Cu) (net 3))
 (segment (start 52.6565 155.2788) (end 52.6565 156.972) (width 0.25) (layer F.Cu) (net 3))
 (segment (start 63.0485 157.888) (end 62.484 157.3235) (width 0.25) (layer F.Cu) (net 3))
 (segment (start 64.516 157.3235) (end 63.613 157.3235) (width 0.25) (layer F.Cu) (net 3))
 (segment (start 63.613 157.3235) (end 63.0485 157.888) (width 0.25) (layer F.Cu) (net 3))
 (segment (start 62.913 158.8847) (end 63.0485 158.7492) (width 0.25) (layer F.Cu) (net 3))
 (segment (start 63.0485 158.7492) (end 63.0485 157.888) (width 0.25) (layer F.Cu) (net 3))
 (segment (start 62.913 159.91) (end 62.913 158.8847) (width 0.25) (layer F.Cu) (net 3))
 (segment (start 62.913 159.91) (end 62.913 160.2103) (width 0.25) (layer F.Cu) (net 3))
 (segment (start 62.913 160.2103) (end 63.0327 160.33) (width 0.25) (layer F.Cu) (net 3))
 (segment (start 63.0327 160.33) (end 63.0327 160.99) (width 0.25) (layer F.Cu) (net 3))
 (segment (start 63.0327 160.99) (end 62.738 161.2847) (width 0.25) (layer F.Cu) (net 3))
 (segment (start 62.738 162.56) (end 62.738 161.2847) (width 0.25) (layer F.Cu) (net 3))
 (segment (start 60.488 162.56) (end 62.738 162.56) (width 0.25) (layer F.Cu) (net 3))
 (segment (start 59.69 157.2255) (end 57.658 157.2255) (width 0.25) (layer F.Cu) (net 3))
 (segment (start 52.832 154.178) (end 52.832 155.1033) (width 0.25) (layer F.Cu) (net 3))
 (segment (start 63.933 160.33) (end 63.933 161.3803) (width 0.25) (layer F.Cu) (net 3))
 (segment (start 65.188 162.56) (end 64.0083 161.3803) (width 0.25) (layer F.Cu) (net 3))
 (segment (start 64.0083 161.3803) (end 63.933 161.3803) (width 0.25) (layer F.Cu) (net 3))
 (segment (start 63.933 160.33) (end 63.0327 160.33) (width 0.25) (layer F.Cu) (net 3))
 (segment (start 66.137 153.67) (end 67.9886 151.8184) (width 0.25) (layer F.Cu) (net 1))
 (segment (start 67.9886 151.8184) (end 67.9886 150.4086) (width 0.25) (layer F.Cu) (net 1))
 (segment (start 67.9886 150.4086) (end 67.404 149.824) (width 0.25) (layer F.Cu) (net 1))
 (segment (start 67.404 149.824) (end 66.172 149.824) (width 0.25) (layer F.Cu) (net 1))
 (segment (start 66.137 153.67) (end 66.137 153.8275) (width 0.25) (layer F.Cu) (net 1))
 (segment (start 66.137 153.8275) (end 64.516 155.4485) (width 0.25) (layer F.Cu) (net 1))
 (segment (start 52.324 144.272) (end 50.9038 145.6922) (width 0.25) (layer F.Cu) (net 1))
 (segment (start 50.9038 145.6922) (end 50.9038 150.4409) (width 0.25) (layer F.Cu) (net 1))
 (segment (start 50.9038 150.4409) (end 50.292 151.0527) (width 0.25) (layer F.Cu) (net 1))
 (segment (start 58.3127 145.6739) (end 59.189 144.7976) (width 0.25) (layer B.Cu) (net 1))
 (segment (start 59.189 144.7976) (end 59.189 144.4709) (width 0.25) (layer B.Cu) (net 1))
 (segment (start 64.516 155.4485) (end 66.4782 157.4107) (width 0.25) (layer F.Cu) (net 1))
 (segment (start 66.4782 157.4107) (end 66.4782 163.0459) (width 0.25) (layer F.Cu) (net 1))
 (segment (start 66.4782 163.0459) (end 65.6597 163.8644) (width 0.25) (layer F.Cu) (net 1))
 (segment (start 65.6597 163.8644) (end 51.4154 163.8644) (width 0.25) (layer F.Cu) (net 1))
 (segment (start 51.4154 163.8644) (end 48.6083 161.0573) (width 0.25) (layer F.Cu) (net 1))
 (segment (start 48.6083 161.0573) (end 48.6083 154.081) (width 0.25) (layer F.Cu) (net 1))
 (segment (start 48.6083 154.081) (end 49.786 152.9033) (width 0.25) (layer F.Cu) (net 1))
 (segment (start 49.786 152.9033) (end 50.292 152.9033) (width 0.25) (layer F.Cu) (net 1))
 (segment (start 50.292 151.978) (end 50.292 152.9033) (width 0.25) (layer F.Cu) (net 1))
 (segment (start 60.972 143.8743) (end 61.4217 144.324) (width 0.25) (layer F.Cu) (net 1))
 (segment (start 61.4217 144.324) (end 66.172 144.324) (width 0.25) (layer F.Cu) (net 1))
 (segment (start 60.972 143.7617) (end 60.972 143.8743) (width 0.25) (layer F.Cu) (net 1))
 (segment (start 60.972 143.124) (end 60.972 143.7617) (width 0.25) (layer F.Cu) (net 1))
 (segment (start 50.292 151.978) (end 50.292 151.0527) (width 0.25) (layer F.Cu) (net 1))
 (segment (start 57.658 155.3505) (end 59.69 155.3505) (width 0.25) (layer F.Cu) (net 1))
 (segment (start 59.472 152.7743) (end 58.835 153.4113) (width 0.25) (layer F.Cu) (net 1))
 (segment (start 58.835 153.4113) (end 56.556 153.4113) (width 0.25) (layer F.Cu) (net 1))
 (segment (start 56.556 153.4113) (end 53.703 156.2643) (width 0.25) (layer F.Cu) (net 1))
 (segment (start 53.703 156.2643) (end 53.703 157.7001) (width 0.25) (layer F.Cu) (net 1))
 (segment (start 53.703 157.7001) (end 54.0075 158.0046) (width 0.25) (layer F.Cu) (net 1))
 (segment (start 54.0075 158.0046) (end 55.0039 158.0046) (width 0.25) (layer F.Cu) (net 1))
 (segment (start 55.0039 158.0046) (end 57.658 155.3505) (width 0.25) (layer F.Cu) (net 1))
 (segment (start 58.0223 147.324) (end 58.0223 145.9643) (width 0.25) (layer F.Cu) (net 1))
 (segment (start 58.0223 145.9643) (end 58.3127 145.6739) (width 0.25) (layer F.Cu) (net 1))
 (segment (start 57.272 147.324) (end 58.0223 147.324) (width 0.25) (layer F.Cu) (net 1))
 (segment (start 59.472 151.2737) (end 58.0223 149.824) (width 0.25) (layer F.Cu) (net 1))
 (segment (start 58.0223 149.824) (end 58.0223 147.324) (width 0.25) (layer F.Cu) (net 1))
 (segment (start 57.272 147.324) (end 56.5217 147.324) (width 0.25) (layer F.Cu) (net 1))
 (segment (start 56.5217 147.324) (end 56.5217 144.5376) (width 0.25) (layer F.Cu) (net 1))
 (segment (start 56.5217 144.5376) (end 56.7353 144.324) (width 0.25) (layer F.Cu) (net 1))
 (segment (start 56.7353 144.324) (end 57.272 144.324) (width 0.25) (layer F.Cu) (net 1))
 (segment (start 59.189 144.4709) (end 59.7856 143.8743) (width 0.25) (layer F.Cu) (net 1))
 (segment (start 59.7856 143.8743) (end 60.972 143.8743) (width 0.25) (layer F.Cu) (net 1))
 (segment (start 52.324 144.272) (end 58.9901 144.272) (width 0.25) (layer B.Cu) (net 1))
 (segment (start 58.9901 144.272) (end 59.189 144.4709) (width 0.25) (layer B.Cu) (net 1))
 (segment (start 59.472 152.024) (end 59.472 151.2737) (width 0.25) (layer F.Cu) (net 1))
 (segment (start 62.484 155.4485) (end 61.972 154.9365) (width 0.25) (layer F.Cu) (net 1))
 (segment (start 61.972 154.9365) (end 61.972 152.024) (width 0.25) (layer F.Cu) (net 1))
 (segment (start 64.516 155.4485) (end 62.484 155.4485) (width 0.25) (layer F.Cu) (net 1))
 (segment (start 59.472 152.024) (end 59.472 152.7743) (width 0.25) (layer F.Cu) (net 1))
 (via (at 58.3127 145.6739) (size 0.8) (layers F.Cu B.Cu) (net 1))
 (via (at 59.189 144.4709) (size 0.8) (layers F.Cu B.Cu) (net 1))
 (segment (start 66.172 147.824) (end 66.844 147.824) (width 0.25) (layer F.Cu) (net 14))
 (segment (start 66.844 147.824) (end 67.3821 147.2859) (width 0.25) (layer F.Cu) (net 14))
 (segment (start 67.3821 147.2859) (end 67.3821 141.7105) (width 0.25) (layer F.Cu) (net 14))
 (segment (start 67.3821 141.7105) (end 65.4065 139.7349) (width 0.25) (layer F.Cu) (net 14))
 (segment (start 65.4065 139.7349) (end 51.8269 139.7349) (width 0.25) (layer F.Cu) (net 14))
 (segment (start 51.8269 139.7349) (end 48.9377 142.6241) (width 0.25) (layer F.Cu) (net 14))
 (segment (start 48.9377 142.6241) (end 48.9377 145.9657) (width 0.25) (layer F.Cu) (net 14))
 (segment (start 48.9377 145.9657) (end 49.784 146.812) (width 0.25) (layer F.Cu) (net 14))
 (segment (start 66.9223 148.324) (end 66.9809 148.324) (width 0.25) (layer F.Cu) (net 12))
 (segment (start 66.9809 148.324) (end 67.8325 147.4724) (width 0.25) (layer F.Cu) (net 12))
 (segment (start 67.8325 147.4724) (end 67.8325 141.524) (width 0.25) (layer F.Cu) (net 12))
 (segment (start 67.8325 141.524) (end 65.593 139.2845) (width 0.25) (layer F.Cu) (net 12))
 (segment (start 65.593 139.2845) (end 51.6404 139.2845) (width 0.25) (layer F.Cu) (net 12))
 (segment (start 51.6404 139.2845) (end 48.4299 142.495) (width 0.25) (layer F.Cu) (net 12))
 (segment (start 48.4299 142.495) (end 48.4299 146.7279) (width 0.25) (layer F.Cu) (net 12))
 (segment (start 48.4299 146.7279) (end 49.784 148.082) (width 0.25) (layer F.Cu) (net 12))
 (segment (start 66.172 148.324) (end 66.9223 148.324) (width 0.25) (layer F.Cu) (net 12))
 (segment (start 66.172 150.824) (end 65.3894 150.824) (width 0.25) (layer F.Cu) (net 16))
 (segment (start 65.3894 150.824) (end 65.1012 150.5358) (width 0.25) (layer F.Cu) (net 16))
 (segment (start 52.324 145.542) (end 53.243 146.461) (width 0.25) (layer B.Cu) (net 16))
 (segment (start 53.243 146.461) (end 61.0264 146.461) (width 0.25) (layer B.Cu) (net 16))
 (segment (start 61.0264 146.461) (end 65.1012 150.5358) (width 0.25) (layer B.Cu) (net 16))
 (via (at 65.1012 150.5358) (size 0.8) (layers F.Cu B.Cu) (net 16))
 (segment (start 66.172 151.324) (end 66.9223 151.324) (width 0.25) (layer F.Cu) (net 17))
 (segment (start 66.9223 151.324) (end 66.9223 151.0318) (width 0.25) (layer F.Cu) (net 17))
 (segment (start 66.9223 151.0318) (end 67.2361 150.718) (width 0.25) (layer F.Cu) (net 17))
 (segment (start 49.784 143.002) (end 50.6179 142.1681) (width 0.25) (layer B.Cu) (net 17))
 (segment (start 50.6179 142.1681) (end 58.6862 142.1681) (width 0.25) (layer B.Cu) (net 17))
 (segment (start 58.6862 142.1681) (end 67.2361 150.718) (width 0.25) (layer B.Cu) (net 17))
 (via (at 67.2361 150.718) (size 0.8) (layers F.Cu B.Cu) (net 17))
 (segment (start 65.472 152.024) (end 66.161 152.024) (width 0.25) (layer F.Cu) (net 18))
 (segment (start 66.161 152.024) (end 66.235 152.098) (width 0.25) (layer F.Cu) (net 18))
 (segment (start 52.324 143.002) (end 58.8126 143.002) (width 0.25) (layer B.Cu) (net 18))
 (segment (start 58.8126 143.002) (end 66.235 150.4244) (width 0.25) (layer B.Cu) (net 18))
 (segment (start 66.235 150.4244) (end 66.235 152.098) (width 0.25) (layer B.Cu) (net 18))
 (via (at 66.235 152.098) (size 0.8) (layers F.Cu B.Cu) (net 18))
 (segment (start 66.172 149.324) (end 64.9663 149.324) (width 0.25) (layer F.Cu) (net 15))
 (segment (start 64.9663 149.324) (end 63.912 150.3783) (width 0.25) (layer F.Cu) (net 15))
 (segment (start 52.324 146.812) (end 52.7686 147.2566) (width 0.25) (layer B.Cu) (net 15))
 (segment (start 52.7686 147.2566) (end 60.7903 147.2566) (width 0.25) (layer B.Cu) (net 15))
 (segment (start 60.7903 147.2566) (end 63.912 150.3783) (width 0.25) (layer B.Cu) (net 15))
 (via (at 63.912 150.3783) (size 0.8) (layers F.Cu B.Cu) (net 15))
 (segment (start 53.4993 160.528) (end 53.8706 160.528) (width 0.25) (layer F.Cu) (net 8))
 (segment (start 53.8706 160.528) (end 55.5139 158.8847) (width 0.25) (layer F.Cu) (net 8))
 (segment (start 55.5139 158.8847) (end 60.313 158.8847) (width 0.25) (layer F.Cu) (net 8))
 (segment (start 60.313 159.91) (end 60.313 158.8847) (width 0.25) (layer F.Cu) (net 8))
 (segment (start 52.324 160.528) (end 53.4993 160.528) (width 0.25) (layer F.Cu) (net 8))
 (segment (start 56.2219 148.079) (end 58.1417 148.079) (width 0.25) (layer B.Cu) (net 11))
 (segment (start 58.1417 148.079) (end 63.1142 153.0515) (width 0.25) (layer B.Cu) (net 11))
 (segment (start 63.472 142.349) (end 63.472 141.252) (width 0.25) (layer F.Cu) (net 11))
 (segment (start 63.472 141.252) (end 63.5 141.224) (width 0.25) (layer F.Cu) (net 11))
 (segment (start 63.472 143.124) (end 63.472 142.349) (width 0.25) (layer F.Cu) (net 11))
 (segment (start 56.8969 143.824) (end 56.8969 143.0987) (width 0.25) (layer F.Cu) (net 11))
 (segment (start 56.8969 143.0987) (end 57.6466 142.349) (width 0.25) (layer F.Cu) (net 11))
 (segment (start 57.6466 142.349) (end 63.472 142.349) (width 0.25) (layer F.Cu) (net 11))
 (segment (start 56.8969 143.824) (end 56.5217 143.824) (width 0.25) (layer F.Cu) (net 11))
 (segment (start 57.272 143.824) (end 56.8969 143.824) (width 0.25) (layer F.Cu) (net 11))
 (segment (start 56.2219 148.079) (end 56.0557 147.9128) (width 0.25) (layer F.Cu) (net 11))
 (segment (start 56.0557 147.9128) (end 56.0557 144.29) (width 0.25) (layer F.Cu) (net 11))
 (segment (start 56.0557 144.29) (end 56.5217 143.824) (width 0.25) (layer F.Cu) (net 11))
 (segment (start 56.5217 151.324) (end 56.2219 151.0242) (width 0.25) (layer F.Cu) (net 11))
 (segment (start 56.2219 151.0242) (end 56.2219 148.079) (width 0.25) (layer F.Cu) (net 11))
 (segment (start 63.1142 153.0515) (end 63.3914 152.7743) (width 0.25) (layer F.Cu) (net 11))
 (segment (start 63.3914 152.7743) (end 63.472 152.7743) (width 0.25) (layer F.Cu) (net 11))
 (segment (start 63.472 152.024) (end 63.472 152.7743) (width 0.25) (layer F.Cu) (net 11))
 (segment (start 57.272 151.324) (end 56.5217 151.324) (width 0.25) (layer F.Cu) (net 11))
 (via (at 63.1142 153.0515) (size 0.8) (layers F.Cu B.Cu) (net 11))
 (via (at 56.2219 148.079) (size 0.8) (layers F.Cu B.Cu) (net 11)))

